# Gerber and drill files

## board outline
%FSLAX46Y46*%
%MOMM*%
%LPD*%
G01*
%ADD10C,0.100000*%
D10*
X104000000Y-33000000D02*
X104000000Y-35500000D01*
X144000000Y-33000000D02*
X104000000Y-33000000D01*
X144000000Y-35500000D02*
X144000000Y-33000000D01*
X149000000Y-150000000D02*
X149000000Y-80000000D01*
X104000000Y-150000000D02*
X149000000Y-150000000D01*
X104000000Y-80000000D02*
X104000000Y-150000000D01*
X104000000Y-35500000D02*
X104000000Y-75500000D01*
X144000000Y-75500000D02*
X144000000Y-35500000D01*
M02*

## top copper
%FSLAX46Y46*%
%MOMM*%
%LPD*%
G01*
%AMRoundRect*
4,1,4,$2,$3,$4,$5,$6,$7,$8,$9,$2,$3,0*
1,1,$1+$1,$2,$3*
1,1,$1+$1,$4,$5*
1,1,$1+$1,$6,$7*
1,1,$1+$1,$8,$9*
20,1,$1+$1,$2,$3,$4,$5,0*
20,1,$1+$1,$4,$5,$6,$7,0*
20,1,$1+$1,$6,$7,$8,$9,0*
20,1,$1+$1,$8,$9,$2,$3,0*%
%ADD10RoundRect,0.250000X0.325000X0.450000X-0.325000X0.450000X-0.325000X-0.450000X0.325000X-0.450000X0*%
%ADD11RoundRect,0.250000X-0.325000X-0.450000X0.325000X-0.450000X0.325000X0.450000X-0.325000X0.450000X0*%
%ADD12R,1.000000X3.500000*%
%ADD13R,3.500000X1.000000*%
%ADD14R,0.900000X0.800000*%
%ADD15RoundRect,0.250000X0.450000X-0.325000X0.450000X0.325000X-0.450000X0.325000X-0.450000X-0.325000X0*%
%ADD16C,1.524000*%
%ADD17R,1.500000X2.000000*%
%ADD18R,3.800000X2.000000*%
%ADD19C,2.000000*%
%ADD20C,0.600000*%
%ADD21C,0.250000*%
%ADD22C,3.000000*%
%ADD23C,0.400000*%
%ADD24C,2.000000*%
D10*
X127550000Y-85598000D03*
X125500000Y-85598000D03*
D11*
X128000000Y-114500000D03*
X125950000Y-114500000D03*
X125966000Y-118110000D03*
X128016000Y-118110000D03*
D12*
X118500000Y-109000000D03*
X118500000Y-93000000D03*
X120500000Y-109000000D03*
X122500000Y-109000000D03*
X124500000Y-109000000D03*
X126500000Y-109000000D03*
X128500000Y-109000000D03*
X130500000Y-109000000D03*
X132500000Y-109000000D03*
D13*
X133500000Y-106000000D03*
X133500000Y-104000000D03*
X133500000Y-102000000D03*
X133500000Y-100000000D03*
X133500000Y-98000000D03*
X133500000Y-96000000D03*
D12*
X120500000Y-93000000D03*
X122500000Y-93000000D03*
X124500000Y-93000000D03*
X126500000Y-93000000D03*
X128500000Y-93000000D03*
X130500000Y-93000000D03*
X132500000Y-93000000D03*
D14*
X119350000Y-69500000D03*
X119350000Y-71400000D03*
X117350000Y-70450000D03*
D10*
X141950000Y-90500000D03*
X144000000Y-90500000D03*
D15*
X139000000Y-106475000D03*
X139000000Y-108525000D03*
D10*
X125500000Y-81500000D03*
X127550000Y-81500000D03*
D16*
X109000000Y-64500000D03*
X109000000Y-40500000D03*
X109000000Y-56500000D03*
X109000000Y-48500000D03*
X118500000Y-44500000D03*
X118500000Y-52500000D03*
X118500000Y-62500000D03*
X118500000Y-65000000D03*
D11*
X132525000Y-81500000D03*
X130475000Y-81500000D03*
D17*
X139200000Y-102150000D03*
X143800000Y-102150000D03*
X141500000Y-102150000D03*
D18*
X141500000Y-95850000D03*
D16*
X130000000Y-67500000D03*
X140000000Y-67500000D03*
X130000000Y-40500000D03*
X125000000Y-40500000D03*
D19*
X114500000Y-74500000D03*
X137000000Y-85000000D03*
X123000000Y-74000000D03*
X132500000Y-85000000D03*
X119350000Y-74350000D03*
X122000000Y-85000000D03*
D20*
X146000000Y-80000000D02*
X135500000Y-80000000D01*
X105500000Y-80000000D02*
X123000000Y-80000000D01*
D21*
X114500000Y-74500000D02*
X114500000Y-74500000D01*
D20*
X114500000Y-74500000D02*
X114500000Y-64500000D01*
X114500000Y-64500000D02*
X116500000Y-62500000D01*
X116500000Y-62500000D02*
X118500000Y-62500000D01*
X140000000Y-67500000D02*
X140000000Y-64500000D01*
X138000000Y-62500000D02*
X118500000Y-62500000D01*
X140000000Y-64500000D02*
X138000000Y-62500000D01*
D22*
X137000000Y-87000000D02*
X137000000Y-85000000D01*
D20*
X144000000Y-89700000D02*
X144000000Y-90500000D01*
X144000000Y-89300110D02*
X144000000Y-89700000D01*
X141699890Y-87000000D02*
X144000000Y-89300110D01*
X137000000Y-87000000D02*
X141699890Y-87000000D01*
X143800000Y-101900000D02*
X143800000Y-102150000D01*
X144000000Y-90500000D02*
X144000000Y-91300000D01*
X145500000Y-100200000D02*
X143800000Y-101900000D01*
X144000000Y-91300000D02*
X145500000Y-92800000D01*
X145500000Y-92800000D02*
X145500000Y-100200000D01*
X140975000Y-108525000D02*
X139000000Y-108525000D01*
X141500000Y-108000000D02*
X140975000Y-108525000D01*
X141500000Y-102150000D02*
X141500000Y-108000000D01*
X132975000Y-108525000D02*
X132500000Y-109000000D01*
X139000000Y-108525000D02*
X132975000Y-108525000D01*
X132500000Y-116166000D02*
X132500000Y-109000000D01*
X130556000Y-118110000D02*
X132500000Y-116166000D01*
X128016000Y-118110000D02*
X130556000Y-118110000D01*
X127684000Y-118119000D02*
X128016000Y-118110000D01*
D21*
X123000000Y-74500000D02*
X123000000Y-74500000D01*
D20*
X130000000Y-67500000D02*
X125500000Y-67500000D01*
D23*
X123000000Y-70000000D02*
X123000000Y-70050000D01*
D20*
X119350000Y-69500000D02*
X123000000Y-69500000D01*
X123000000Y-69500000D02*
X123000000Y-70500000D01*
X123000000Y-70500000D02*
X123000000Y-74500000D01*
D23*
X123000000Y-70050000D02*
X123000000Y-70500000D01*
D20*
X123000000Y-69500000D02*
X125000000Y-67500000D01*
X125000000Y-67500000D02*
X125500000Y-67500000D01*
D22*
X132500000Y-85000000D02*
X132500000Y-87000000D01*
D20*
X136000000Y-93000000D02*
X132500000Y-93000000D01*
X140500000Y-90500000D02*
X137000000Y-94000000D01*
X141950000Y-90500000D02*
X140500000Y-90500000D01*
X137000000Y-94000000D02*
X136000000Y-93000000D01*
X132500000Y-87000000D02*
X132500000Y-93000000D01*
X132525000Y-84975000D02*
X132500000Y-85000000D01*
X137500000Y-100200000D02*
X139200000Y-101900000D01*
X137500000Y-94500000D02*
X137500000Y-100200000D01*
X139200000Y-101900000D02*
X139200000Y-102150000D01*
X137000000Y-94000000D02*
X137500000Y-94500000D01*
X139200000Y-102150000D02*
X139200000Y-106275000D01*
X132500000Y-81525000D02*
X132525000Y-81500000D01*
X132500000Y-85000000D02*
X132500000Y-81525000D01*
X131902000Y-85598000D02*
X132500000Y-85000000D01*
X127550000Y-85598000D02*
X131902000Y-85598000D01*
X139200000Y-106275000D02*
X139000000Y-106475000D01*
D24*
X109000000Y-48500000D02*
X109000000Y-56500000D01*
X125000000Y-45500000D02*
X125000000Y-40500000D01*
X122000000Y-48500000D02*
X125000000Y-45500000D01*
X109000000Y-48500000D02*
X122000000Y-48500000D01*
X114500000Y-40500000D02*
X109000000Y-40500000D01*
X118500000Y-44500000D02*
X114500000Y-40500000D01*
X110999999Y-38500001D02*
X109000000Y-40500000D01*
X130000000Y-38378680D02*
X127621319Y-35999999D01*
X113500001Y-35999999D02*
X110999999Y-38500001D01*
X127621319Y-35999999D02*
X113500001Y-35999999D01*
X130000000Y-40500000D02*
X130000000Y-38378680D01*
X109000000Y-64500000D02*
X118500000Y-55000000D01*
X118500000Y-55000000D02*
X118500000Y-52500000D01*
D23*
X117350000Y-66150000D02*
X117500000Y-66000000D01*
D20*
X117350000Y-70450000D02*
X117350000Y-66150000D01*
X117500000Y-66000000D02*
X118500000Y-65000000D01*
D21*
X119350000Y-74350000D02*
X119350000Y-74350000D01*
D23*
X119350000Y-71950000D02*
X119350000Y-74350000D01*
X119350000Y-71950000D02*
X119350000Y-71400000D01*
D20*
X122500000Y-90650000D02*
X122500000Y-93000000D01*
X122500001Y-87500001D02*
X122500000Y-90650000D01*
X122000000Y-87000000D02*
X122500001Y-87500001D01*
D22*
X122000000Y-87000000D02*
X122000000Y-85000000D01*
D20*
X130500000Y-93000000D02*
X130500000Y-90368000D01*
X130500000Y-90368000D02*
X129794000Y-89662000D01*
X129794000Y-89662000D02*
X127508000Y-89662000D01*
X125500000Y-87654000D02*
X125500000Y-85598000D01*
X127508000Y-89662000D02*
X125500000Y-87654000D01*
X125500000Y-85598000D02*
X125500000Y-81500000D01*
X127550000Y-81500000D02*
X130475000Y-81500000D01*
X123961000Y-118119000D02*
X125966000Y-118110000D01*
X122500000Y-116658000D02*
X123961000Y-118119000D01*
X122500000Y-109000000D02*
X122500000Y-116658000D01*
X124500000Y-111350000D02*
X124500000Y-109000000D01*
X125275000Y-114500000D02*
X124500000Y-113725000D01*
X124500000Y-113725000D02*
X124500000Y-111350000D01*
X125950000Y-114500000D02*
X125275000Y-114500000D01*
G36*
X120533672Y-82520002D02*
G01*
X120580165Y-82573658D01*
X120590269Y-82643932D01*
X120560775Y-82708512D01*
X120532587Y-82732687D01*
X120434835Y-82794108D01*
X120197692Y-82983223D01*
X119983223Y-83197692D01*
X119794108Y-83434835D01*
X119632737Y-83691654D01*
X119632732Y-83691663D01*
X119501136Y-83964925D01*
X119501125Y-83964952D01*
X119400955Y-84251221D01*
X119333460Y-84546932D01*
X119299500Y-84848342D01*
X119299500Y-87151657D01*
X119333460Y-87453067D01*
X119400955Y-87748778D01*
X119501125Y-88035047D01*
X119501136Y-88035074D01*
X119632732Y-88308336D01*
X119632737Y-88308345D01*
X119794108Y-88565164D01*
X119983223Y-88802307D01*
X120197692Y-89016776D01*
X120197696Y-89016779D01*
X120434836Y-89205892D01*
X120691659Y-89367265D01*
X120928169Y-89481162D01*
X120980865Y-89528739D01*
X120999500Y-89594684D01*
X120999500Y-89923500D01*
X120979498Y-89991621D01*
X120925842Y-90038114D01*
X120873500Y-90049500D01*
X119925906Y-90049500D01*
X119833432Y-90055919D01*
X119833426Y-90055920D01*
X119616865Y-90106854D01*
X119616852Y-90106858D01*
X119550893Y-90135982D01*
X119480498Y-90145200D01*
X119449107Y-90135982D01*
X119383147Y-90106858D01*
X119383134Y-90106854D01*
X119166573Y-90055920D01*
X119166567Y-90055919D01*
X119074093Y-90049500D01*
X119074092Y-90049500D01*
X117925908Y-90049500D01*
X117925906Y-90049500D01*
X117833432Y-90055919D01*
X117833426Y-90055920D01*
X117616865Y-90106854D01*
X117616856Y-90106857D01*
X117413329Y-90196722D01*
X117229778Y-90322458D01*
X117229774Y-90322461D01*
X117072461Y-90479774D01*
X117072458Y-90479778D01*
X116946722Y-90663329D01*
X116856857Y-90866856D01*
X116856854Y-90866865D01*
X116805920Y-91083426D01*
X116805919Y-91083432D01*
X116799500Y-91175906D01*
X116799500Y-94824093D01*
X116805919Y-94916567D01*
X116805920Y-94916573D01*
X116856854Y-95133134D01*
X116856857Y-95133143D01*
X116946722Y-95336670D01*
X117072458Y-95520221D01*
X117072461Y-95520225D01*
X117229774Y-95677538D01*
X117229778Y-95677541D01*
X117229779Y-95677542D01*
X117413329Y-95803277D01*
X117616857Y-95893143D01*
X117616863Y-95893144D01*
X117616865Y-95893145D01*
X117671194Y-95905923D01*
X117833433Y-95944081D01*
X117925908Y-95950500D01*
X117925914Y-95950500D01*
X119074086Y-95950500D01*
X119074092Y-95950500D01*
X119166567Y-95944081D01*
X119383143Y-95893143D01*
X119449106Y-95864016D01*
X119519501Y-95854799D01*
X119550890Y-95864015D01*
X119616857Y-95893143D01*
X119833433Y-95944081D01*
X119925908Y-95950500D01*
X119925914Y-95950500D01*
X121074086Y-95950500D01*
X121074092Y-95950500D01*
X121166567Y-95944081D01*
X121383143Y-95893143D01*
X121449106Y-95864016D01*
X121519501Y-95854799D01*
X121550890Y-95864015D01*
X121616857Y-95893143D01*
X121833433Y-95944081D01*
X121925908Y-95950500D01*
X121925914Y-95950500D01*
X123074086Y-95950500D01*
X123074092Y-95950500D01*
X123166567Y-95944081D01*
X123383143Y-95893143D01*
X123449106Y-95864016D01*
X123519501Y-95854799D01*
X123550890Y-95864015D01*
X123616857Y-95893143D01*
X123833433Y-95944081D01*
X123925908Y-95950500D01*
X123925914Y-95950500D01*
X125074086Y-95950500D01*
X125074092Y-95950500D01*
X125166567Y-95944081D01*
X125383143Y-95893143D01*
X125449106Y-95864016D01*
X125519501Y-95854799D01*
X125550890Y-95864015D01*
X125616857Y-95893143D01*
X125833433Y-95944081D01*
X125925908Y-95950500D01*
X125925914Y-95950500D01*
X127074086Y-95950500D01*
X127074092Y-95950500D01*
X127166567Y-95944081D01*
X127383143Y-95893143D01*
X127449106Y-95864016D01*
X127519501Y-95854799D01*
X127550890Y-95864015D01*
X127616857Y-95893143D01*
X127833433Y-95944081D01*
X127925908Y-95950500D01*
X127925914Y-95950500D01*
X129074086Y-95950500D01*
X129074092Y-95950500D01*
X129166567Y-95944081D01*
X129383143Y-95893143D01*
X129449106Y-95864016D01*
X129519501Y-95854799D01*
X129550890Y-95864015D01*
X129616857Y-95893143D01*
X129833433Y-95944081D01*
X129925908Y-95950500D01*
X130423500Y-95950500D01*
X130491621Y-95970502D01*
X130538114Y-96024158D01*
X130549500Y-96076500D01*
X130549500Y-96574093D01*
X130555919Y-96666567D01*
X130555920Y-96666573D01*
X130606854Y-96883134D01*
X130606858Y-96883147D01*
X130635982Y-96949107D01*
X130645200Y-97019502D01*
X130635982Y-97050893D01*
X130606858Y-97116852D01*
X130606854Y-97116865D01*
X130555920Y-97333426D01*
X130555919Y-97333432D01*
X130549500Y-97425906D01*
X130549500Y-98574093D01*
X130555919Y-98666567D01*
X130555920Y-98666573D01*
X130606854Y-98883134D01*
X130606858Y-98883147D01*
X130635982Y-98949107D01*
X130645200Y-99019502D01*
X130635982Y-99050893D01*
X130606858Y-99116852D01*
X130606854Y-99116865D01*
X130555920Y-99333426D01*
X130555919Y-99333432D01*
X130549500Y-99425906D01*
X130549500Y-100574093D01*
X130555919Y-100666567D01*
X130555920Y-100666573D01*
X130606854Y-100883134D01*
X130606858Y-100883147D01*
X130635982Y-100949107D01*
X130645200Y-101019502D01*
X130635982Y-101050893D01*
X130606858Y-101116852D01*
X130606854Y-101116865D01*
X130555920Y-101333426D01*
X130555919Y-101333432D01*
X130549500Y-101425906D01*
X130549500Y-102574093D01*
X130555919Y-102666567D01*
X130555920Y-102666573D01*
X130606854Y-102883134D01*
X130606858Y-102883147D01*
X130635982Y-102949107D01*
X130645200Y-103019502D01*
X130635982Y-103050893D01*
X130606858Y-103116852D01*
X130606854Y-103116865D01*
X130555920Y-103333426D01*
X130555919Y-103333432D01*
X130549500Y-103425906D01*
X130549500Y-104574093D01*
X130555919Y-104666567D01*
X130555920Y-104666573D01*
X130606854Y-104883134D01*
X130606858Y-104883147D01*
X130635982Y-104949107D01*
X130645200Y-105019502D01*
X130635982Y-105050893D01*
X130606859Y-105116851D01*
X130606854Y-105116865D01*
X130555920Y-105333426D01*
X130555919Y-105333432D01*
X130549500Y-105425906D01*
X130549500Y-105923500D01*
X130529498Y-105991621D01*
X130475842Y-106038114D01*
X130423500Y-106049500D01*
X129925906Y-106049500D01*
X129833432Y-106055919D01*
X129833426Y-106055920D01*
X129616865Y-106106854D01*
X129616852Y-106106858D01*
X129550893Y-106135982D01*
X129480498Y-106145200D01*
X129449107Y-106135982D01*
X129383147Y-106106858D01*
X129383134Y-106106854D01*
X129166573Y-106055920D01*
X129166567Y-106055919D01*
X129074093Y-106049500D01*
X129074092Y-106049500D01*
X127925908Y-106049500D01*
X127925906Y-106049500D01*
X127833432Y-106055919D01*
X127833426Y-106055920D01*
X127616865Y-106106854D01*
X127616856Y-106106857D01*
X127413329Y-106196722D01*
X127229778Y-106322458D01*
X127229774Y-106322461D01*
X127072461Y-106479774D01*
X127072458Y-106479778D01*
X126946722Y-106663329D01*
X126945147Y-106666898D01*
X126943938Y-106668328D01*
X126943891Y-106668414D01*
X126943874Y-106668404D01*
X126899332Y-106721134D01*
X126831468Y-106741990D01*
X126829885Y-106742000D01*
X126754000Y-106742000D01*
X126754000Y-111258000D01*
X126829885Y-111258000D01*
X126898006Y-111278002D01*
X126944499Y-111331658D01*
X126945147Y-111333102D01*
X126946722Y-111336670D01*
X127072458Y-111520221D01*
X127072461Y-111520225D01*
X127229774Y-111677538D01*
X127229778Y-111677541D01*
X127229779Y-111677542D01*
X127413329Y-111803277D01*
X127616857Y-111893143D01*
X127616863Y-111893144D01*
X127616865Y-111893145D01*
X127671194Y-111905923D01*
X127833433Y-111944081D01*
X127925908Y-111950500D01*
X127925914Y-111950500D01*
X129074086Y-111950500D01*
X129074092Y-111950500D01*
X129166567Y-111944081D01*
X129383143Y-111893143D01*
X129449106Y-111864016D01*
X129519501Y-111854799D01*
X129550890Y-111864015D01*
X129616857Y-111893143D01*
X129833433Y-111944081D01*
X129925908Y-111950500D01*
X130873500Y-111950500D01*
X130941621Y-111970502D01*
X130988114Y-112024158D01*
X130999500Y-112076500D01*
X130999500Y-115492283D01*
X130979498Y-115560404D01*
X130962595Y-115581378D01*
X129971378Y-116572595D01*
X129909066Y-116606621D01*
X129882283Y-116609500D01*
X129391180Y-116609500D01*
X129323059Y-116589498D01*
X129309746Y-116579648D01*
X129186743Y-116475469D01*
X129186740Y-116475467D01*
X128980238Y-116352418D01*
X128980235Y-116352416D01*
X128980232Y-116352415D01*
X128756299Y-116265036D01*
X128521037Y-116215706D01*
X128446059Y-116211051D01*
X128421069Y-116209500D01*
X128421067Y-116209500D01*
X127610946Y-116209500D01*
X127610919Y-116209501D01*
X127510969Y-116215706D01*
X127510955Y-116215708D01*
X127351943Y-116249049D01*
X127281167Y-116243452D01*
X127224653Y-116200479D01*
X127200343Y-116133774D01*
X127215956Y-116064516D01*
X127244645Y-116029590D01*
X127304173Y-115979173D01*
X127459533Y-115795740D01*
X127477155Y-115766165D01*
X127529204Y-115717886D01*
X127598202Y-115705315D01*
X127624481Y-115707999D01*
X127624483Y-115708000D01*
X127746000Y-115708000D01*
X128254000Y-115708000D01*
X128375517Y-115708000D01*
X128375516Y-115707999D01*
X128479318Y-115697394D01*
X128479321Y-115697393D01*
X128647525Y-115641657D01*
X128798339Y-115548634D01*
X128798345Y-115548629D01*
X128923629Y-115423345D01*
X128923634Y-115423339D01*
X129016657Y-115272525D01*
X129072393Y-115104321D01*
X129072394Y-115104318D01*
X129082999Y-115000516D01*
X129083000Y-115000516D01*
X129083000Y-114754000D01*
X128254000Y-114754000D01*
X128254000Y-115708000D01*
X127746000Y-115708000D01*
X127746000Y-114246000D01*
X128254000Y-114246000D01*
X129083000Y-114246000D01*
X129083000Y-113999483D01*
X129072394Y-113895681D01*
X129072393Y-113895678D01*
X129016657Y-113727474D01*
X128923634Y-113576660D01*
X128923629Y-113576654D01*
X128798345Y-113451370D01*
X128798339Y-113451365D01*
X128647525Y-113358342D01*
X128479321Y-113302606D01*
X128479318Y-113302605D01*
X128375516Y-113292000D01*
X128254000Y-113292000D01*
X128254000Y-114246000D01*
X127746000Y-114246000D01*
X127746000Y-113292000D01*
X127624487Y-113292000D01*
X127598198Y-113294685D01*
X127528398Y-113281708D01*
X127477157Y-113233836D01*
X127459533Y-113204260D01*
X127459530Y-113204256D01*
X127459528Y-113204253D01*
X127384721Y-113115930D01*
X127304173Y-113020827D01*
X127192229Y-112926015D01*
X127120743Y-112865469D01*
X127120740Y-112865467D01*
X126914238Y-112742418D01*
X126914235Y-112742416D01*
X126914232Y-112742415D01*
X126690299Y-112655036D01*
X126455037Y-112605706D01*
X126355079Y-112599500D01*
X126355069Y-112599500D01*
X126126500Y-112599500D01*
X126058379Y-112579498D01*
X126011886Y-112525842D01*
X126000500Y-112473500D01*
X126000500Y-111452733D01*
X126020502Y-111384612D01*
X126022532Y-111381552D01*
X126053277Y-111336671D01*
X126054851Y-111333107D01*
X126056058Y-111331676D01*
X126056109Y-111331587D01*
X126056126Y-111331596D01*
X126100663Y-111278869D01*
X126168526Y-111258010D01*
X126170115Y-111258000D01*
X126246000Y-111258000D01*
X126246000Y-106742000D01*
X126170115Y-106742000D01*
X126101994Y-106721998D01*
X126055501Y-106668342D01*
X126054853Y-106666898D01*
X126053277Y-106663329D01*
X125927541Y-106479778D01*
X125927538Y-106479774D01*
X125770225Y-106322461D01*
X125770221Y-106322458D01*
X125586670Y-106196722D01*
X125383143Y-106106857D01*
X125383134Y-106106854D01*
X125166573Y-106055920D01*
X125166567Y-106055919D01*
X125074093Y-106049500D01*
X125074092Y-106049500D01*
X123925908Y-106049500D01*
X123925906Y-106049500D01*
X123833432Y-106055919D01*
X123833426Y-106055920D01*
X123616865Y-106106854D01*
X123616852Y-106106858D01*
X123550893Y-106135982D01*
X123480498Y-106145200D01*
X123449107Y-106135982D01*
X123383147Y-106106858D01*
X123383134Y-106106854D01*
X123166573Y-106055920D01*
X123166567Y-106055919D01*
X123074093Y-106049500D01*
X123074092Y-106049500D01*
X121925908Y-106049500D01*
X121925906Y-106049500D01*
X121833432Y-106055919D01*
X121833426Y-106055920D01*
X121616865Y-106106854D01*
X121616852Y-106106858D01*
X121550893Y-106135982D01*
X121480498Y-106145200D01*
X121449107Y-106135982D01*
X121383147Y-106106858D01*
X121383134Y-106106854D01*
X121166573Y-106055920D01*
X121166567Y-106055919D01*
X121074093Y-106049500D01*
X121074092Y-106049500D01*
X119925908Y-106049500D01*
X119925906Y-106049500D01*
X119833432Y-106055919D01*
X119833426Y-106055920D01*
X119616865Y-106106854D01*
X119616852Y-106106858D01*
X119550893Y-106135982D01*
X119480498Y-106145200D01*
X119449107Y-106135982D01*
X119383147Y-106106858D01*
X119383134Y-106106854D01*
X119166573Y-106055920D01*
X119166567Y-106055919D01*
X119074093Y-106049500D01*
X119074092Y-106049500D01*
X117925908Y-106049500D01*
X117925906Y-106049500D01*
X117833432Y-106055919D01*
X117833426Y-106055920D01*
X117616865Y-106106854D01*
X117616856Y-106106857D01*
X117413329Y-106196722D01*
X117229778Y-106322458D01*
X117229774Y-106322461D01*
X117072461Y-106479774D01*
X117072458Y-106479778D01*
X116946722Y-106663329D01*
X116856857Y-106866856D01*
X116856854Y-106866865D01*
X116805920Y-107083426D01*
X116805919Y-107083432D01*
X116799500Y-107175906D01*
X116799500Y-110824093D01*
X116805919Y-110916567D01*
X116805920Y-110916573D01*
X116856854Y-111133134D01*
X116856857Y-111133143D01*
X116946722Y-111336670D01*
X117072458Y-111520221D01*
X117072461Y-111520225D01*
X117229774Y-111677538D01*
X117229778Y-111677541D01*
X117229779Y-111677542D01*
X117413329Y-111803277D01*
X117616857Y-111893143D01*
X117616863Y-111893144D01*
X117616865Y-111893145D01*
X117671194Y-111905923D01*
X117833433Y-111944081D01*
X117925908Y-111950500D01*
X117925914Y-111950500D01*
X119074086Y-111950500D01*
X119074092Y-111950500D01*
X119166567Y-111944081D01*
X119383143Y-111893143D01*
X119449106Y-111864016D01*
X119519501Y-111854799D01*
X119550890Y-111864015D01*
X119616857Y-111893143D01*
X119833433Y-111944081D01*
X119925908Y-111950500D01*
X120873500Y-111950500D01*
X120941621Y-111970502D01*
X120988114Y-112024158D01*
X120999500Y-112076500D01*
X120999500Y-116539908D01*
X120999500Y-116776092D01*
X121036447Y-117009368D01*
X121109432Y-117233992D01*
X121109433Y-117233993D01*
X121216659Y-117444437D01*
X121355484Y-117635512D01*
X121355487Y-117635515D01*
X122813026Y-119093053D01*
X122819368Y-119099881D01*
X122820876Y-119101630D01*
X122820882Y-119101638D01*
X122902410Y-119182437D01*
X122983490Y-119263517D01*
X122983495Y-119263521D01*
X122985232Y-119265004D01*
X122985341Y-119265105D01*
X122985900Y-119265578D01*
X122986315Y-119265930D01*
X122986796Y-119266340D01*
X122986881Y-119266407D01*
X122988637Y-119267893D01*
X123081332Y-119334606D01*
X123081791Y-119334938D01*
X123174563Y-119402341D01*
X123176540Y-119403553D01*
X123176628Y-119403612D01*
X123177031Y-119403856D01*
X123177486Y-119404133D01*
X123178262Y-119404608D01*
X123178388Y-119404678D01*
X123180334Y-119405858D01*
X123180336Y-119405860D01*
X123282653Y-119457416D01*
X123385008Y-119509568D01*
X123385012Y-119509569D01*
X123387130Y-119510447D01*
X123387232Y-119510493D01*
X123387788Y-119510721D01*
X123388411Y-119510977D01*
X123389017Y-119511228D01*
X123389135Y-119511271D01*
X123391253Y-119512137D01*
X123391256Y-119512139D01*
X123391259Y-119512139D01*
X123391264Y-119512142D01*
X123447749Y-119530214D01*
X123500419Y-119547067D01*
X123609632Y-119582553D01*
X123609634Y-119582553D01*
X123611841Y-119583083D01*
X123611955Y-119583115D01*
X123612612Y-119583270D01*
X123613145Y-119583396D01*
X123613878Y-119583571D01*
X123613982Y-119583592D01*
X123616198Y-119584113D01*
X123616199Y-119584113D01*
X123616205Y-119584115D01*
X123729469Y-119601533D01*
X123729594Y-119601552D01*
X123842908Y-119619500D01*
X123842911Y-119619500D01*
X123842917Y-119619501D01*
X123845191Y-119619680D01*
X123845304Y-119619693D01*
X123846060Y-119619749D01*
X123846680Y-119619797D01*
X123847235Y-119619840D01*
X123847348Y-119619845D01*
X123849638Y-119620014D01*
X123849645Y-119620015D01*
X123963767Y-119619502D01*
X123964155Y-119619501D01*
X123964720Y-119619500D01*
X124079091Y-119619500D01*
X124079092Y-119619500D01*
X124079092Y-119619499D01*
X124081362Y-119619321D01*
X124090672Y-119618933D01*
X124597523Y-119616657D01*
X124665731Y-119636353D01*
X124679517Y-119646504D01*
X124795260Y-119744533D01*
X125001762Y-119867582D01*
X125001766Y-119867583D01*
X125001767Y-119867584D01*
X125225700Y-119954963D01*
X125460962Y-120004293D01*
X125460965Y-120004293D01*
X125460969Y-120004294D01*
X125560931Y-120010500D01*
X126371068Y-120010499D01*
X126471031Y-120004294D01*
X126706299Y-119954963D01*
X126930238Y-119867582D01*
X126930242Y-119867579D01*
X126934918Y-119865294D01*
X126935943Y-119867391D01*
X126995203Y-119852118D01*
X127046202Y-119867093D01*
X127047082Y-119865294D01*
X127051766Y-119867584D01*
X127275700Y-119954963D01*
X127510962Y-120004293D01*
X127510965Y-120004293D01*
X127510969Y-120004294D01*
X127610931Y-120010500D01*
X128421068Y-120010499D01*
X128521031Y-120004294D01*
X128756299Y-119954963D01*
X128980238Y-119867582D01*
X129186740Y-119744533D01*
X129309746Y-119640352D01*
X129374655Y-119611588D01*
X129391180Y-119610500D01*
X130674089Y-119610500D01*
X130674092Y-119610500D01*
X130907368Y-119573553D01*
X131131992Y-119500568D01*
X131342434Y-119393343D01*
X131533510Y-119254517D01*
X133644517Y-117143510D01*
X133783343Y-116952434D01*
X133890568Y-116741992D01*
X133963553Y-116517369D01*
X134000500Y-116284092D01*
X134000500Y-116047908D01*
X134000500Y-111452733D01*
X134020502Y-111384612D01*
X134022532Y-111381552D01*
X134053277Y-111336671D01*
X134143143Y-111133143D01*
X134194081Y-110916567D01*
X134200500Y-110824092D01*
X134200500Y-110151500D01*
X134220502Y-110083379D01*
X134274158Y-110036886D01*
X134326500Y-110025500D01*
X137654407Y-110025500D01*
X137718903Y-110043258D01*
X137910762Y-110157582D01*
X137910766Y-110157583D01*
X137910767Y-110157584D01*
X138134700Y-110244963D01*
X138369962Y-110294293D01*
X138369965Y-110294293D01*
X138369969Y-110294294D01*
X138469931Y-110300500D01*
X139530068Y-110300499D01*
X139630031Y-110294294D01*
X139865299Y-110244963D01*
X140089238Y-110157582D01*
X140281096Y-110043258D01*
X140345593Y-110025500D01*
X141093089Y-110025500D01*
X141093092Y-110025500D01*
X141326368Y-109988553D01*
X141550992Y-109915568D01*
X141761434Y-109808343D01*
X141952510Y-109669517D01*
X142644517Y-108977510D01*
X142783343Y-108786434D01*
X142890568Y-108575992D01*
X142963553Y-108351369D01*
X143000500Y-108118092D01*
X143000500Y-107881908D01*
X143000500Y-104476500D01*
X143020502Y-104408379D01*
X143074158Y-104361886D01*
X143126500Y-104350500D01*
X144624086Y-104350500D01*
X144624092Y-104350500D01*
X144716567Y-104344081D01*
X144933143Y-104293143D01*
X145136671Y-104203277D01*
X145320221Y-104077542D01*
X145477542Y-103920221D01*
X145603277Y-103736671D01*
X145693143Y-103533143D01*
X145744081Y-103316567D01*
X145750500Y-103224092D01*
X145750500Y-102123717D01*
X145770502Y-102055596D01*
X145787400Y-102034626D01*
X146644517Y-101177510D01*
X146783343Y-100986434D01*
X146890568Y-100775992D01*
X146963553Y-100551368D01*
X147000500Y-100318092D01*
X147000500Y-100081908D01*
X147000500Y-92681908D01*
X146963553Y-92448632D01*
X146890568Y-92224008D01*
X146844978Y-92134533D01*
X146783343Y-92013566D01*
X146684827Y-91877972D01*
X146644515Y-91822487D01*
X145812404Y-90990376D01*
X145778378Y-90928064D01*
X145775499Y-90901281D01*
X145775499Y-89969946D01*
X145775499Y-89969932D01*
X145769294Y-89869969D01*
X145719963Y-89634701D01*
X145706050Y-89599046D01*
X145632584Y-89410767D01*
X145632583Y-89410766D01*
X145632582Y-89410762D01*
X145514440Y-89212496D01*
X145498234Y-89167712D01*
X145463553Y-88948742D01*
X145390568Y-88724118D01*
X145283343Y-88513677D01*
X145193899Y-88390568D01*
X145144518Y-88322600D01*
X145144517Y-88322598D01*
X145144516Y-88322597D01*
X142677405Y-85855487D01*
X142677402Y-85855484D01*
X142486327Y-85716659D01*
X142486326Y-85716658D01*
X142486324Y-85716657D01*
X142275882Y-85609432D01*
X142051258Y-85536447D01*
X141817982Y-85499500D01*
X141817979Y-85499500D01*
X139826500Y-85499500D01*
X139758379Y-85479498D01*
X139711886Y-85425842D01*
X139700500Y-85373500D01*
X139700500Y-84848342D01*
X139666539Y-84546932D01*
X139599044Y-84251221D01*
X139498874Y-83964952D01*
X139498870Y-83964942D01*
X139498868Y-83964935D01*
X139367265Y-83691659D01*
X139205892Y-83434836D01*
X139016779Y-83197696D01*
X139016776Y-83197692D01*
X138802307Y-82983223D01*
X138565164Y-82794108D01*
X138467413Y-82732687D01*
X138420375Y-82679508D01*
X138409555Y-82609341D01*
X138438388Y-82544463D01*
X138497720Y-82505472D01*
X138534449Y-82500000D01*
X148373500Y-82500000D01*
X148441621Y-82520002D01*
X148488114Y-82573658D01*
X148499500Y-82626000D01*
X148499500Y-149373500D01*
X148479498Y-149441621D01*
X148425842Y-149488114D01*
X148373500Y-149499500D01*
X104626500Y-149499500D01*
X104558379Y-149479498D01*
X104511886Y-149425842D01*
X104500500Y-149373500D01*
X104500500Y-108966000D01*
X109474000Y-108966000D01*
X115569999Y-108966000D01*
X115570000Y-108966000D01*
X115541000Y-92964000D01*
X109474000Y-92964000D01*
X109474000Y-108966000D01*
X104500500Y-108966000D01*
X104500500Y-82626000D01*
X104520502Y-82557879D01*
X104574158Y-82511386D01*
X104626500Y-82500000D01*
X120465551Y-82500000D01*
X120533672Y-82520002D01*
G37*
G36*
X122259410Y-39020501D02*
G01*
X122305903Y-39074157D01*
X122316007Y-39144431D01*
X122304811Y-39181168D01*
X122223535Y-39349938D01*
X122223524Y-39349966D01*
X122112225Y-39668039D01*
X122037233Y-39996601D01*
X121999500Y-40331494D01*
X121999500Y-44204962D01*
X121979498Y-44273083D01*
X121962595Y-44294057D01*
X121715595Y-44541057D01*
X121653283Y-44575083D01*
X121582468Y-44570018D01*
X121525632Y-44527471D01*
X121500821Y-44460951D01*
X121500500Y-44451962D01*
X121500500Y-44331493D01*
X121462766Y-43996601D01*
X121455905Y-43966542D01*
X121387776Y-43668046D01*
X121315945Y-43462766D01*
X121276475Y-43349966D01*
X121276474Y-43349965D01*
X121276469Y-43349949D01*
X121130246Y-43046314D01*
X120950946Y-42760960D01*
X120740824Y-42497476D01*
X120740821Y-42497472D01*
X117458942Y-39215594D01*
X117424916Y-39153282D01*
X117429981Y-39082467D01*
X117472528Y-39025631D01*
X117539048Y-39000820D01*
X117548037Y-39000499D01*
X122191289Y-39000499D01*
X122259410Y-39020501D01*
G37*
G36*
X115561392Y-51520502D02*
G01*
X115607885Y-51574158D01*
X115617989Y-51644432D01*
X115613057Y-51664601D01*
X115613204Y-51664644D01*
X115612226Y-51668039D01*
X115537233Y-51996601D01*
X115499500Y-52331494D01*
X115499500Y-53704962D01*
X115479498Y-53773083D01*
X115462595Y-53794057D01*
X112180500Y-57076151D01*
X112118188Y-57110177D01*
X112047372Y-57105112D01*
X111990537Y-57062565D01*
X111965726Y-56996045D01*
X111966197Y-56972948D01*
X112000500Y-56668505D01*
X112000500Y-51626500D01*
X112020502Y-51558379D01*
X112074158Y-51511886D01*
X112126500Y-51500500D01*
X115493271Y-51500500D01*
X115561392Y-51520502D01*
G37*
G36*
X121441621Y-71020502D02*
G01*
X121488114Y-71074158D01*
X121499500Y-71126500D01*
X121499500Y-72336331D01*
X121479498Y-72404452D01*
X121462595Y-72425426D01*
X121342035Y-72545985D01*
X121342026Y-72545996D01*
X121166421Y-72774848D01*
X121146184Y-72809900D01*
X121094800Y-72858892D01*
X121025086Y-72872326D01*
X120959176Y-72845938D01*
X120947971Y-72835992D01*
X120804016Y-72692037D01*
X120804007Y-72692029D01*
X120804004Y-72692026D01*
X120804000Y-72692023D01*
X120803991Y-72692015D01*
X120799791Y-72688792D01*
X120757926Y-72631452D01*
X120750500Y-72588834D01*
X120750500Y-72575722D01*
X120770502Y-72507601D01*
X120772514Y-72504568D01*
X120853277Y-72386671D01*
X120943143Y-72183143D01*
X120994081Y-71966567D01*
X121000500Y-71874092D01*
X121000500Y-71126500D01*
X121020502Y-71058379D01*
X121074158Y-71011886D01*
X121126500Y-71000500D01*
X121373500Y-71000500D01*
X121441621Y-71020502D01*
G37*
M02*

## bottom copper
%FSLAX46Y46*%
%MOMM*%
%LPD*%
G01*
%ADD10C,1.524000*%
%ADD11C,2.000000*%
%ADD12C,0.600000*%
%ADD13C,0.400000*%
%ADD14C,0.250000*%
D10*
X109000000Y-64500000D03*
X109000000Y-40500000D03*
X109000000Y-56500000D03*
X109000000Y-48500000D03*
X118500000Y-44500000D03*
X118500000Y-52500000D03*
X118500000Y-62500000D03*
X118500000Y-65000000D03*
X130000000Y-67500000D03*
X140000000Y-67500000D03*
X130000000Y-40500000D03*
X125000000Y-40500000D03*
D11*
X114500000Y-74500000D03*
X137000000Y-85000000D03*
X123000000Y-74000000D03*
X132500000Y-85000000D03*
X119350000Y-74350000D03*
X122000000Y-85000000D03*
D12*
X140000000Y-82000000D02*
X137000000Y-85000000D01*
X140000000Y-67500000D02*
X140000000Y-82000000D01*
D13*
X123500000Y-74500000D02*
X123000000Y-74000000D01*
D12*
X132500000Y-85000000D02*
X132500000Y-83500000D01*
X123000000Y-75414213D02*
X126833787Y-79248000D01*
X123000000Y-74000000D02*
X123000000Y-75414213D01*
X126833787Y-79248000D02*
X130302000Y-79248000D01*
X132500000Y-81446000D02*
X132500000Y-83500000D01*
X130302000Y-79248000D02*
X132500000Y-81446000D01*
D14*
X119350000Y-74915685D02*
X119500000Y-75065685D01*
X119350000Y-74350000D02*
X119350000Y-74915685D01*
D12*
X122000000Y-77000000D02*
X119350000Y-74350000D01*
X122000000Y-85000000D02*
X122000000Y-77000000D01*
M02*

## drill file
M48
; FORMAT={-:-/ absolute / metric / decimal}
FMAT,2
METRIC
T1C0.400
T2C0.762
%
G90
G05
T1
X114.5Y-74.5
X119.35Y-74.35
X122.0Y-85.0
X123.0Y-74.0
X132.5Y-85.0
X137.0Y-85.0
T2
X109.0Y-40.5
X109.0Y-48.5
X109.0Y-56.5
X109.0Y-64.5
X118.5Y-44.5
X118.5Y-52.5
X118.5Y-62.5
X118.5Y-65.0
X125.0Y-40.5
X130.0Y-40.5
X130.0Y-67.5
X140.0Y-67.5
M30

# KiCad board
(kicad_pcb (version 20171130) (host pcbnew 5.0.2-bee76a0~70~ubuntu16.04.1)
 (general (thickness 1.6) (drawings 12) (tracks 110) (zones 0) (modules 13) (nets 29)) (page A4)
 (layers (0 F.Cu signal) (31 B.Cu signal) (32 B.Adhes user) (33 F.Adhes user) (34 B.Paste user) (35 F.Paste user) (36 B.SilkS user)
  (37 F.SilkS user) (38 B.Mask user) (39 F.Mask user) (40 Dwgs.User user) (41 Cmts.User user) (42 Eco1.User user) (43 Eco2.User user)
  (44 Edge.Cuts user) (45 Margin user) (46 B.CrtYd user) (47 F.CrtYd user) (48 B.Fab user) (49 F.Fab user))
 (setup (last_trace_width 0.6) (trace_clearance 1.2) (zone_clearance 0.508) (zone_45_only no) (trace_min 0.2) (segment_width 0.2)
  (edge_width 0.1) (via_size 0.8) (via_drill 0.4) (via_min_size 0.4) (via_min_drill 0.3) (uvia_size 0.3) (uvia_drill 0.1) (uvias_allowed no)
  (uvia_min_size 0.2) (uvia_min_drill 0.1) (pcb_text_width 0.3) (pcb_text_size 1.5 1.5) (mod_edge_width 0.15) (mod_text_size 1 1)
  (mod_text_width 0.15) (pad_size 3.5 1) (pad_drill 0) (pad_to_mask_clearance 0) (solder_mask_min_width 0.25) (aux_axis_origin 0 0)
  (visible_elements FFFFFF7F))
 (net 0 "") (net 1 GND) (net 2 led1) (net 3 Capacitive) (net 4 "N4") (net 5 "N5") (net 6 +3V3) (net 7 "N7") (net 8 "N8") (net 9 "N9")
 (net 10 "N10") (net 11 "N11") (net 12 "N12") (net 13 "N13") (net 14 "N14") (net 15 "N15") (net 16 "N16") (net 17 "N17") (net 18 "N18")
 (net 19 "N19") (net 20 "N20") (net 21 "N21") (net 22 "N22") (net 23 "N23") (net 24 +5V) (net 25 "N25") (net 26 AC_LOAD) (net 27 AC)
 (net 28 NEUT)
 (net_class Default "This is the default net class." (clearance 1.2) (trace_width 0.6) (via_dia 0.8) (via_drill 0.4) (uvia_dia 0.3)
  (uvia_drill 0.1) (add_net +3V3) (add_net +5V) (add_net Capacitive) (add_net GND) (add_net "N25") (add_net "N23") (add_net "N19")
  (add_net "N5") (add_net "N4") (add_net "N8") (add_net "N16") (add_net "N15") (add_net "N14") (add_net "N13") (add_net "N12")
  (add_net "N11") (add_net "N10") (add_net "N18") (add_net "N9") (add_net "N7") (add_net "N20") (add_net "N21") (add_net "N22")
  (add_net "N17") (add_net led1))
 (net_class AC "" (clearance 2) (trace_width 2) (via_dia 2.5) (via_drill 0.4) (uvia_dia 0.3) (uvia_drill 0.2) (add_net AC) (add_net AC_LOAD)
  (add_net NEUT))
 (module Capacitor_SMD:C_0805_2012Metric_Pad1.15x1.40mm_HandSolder (layer F.Cu) (at 126.525 85.598 180)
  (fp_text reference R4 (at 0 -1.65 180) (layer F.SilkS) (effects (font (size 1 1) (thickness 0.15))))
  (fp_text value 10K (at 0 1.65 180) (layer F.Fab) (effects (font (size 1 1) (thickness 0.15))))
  (pad 1 smd roundrect (at -1.025 0 180) (size 1.15 1.4) (layers F.Cu F.Paste F.Mask) (roundrect_rratio 0.217391) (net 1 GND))
  (pad 2 smd roundrect (at 1.025 0 180) (size 1.15 1.4) (layers F.Cu F.Paste F.Mask) (roundrect_rratio 0.217391) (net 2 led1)))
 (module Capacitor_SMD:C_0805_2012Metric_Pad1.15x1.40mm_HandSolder (layer F.Cu) (at 126.975 114.5)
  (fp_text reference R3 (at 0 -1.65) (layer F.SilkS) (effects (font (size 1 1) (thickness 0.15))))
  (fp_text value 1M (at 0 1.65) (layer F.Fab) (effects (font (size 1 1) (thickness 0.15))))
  (pad 2 smd roundrect (at 1.025 0) (size 1.15 1.4) (layers F.Cu F.Paste F.Mask) (roundrect_rratio 0.217391) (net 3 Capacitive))
  (pad 1 smd roundrect (at -1.025 0) (size 1.15 1.4) (layers F.Cu F.Paste F.Mask) (roundrect_rratio 0.217391) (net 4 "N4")))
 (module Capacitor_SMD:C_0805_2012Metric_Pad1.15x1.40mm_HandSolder (layer F.Cu) (at 126.991 118.11)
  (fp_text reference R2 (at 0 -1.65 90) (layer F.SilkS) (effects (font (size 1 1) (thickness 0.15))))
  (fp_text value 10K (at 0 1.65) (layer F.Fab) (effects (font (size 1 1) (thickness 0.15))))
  (pad 1 smd roundrect (at -1.025 0) (size 1.15 1.4) (layers F.Cu F.Paste F.Mask) (roundrect_rratio 0.217391) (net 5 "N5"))
  (pad 2 smd roundrect (at 1.025 0) (size 1.15 1.4) (layers F.Cu F.Paste F.Mask) (roundrect_rratio 0.217391) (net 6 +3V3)))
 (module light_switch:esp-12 (layer F.Cu) (at 125.5 101 90)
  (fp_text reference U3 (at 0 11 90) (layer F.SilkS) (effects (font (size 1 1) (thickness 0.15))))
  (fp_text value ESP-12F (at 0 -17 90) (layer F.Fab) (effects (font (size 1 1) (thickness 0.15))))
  (pad 22 smd rect (at -8 -7 90) (size 3.5 1) (layers F.Cu F.Paste F.Mask) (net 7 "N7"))
  (pad 1 smd rect (at 8 -7 90) (size 3.5 1) (layers F.Cu F.Paste F.Mask) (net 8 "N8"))
  (pad 21 smd rect (at -8 -5 90) (size 3.5 1) (layers F.Cu F.Paste F.Mask) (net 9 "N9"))
  (pad 20 smd rect (at -8 -3 90) (size 3.5 1) (layers F.Cu F.Paste F.Mask) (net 5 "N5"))
  (pad 19 smd rect (at -8 -1 90) (size 3.5 1) (layers F.Cu F.Paste F.Mask) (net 4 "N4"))
  (pad 18 smd rect (at -8 1 90) (size 3.5 1) (layers F.Cu F.Paste F.Mask) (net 3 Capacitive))
  (pad 17 smd rect (at -8 3 90) (size 3.5 1) (layers F.Cu F.Paste F.Mask) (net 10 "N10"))
  (pad 16 smd rect (at -8 5 90) (size 3.5 1) (layers F.Cu F.Paste F.Mask) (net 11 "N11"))
  (pad 15 smd rect (at -8 7 90) (size 3.5 1) (layers F.Cu F.Paste F.Mask) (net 6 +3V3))
  (pad 14 smd rect (at -5 8) (size 3.5 1) (layers F.Cu F.Paste F.Mask) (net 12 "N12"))
  (pad 13 smd rect (at -3 8) (size 3.5 1) (layers F.Cu F.Paste F.Mask) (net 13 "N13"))
  (pad 12 smd rect (at -1 8) (size 3.5 1) (layers F.Cu F.Paste F.Mask) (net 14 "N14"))
  (pad 11 smd rect (at 1 8) (size 3.5 1) (layers F.Cu F.Paste F.Mask) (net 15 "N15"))
  (pad 10 smd rect (at 3 8) (size 3.5 1) (layers F.Cu F.Paste F.Mask) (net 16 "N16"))
  (pad 9 smd rect (at 5 8 180) (size 3.5 1) (layers F.Cu F.Paste F.Mask) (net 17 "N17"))
  (pad 2 smd rect (at 8 -5 90) (size 3.5 1) (layers F.Cu F.Paste F.Mask) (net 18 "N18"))
  (pad 3 smd rect (at 8 -3 90) (size 3.5 1) (layers F.Cu F.Paste F.Mask) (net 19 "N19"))
  (pad 4 smd rect (at 8 -1 90) (size 3.5 1) (layers F.Cu F.Paste F.Mask) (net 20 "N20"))
  (pad 5 smd rect (at 8 1 90) (size 3.5 1) (layers F.Cu F.Paste F.Mask) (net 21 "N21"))
  (pad 6 smd rect (at 8 3 90) (size 3.5 1) (layers F.Cu F.Paste F.Mask) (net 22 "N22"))
  (pad 7 smd rect (at 8 5 90) (size 3.5 1) (layers F.Cu F.Paste F.Mask) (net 2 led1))
  (pad 8 smd rect (at 8 7 90) (size 3.5 1) (layers F.Cu F.Paste F.Mask) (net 1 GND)))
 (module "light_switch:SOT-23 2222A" (layer F.Cu) (at 119 70.45 90)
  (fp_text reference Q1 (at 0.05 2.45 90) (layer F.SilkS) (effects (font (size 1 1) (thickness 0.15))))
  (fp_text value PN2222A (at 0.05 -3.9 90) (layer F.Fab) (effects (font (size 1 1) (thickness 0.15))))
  (pad 1 smd rect (at 0.95 0.35 90) (size 0.8 0.9) (layers F.Cu F.Paste F.Mask) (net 1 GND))
  (pad 2 smd rect (at -0.95 0.35 90) (size 0.8 0.9) (layers F.Cu F.Paste F.Mask) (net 19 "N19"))
  (pad 3 smd rect (at 0 -1.65 90) (size 0.8 0.9) (layers F.Cu F.Paste F.Mask) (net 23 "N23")))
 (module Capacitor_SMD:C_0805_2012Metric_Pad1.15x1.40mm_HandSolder (layer F.Cu) (at 142.975 90.5 180)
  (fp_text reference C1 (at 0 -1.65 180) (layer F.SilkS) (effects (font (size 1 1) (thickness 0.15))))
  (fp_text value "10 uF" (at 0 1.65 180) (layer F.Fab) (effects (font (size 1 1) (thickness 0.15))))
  (pad 2 smd roundrect (at 1.025 0 180) (size 1.15 1.4) (layers F.Cu F.Paste F.Mask) (roundrect_rratio 0.217391) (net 1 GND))
  (pad 1 smd roundrect (at -1.025 0 180) (size 1.15 1.4) (layers F.Cu F.Paste F.Mask) (roundrect_rratio 0.217391) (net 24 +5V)))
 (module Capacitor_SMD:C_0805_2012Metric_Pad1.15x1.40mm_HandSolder (layer F.Cu) (at 139 107.5 90)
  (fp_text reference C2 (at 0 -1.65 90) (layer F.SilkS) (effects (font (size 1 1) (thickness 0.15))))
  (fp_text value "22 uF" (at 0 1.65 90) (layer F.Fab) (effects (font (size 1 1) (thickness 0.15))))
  (pad 2 smd roundrect (at 1.025 0 90) (size 1.15 1.4) (layers F.Cu F.Paste F.Mask) (roundrect_rratio 0.217391) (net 1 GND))
  (pad 1 smd roundrect (at -1.025 0 90) (size 1.15 1.4) (layers F.Cu F.Paste F.Mask) (roundrect_rratio 0.217391) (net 6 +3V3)))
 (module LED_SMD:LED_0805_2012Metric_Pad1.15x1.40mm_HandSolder (layer F.Cu) (at 126.525 81.5 180)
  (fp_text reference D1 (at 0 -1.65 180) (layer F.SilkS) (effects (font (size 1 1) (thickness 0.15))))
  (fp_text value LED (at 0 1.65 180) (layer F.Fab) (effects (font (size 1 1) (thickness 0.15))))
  (pad 2 smd roundrect (at 1.025 0 180) (size 1.15 1.4) (layers F.Cu F.Paste F.Mask) (roundrect_rratio 0.217391) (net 2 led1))
  (pad 1 smd roundrect (at -1.025 0 180) (size 1.15 1.4) (layers F.Cu F.Paste F.Mask) (roundrect_rratio 0.217391) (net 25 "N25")))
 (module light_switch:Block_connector (layer F.Cu) (at 109 52.5 270)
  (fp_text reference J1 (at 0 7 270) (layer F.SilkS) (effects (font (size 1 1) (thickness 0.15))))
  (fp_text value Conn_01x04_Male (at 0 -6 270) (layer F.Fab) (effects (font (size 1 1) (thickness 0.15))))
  (pad 4 thru_hole circle (at 12 0 270) (size 1.524 1.524) (drill 0.762) (layers *.Cu *.Mask) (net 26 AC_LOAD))
  (pad 1 thru_hole circle (at -12 0 270) (size 1.524 1.524) (drill 0.762) (layers *.Cu *.Mask) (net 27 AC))
  (pad 3 thru_hole circle (at 4 0 270) (size 1.524 1.524) (drill 0.762) (layers *.Cu *.Mask) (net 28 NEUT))
  (pad 2 thru_hole circle (at -4 0 270) (size 1.524 1.524) (drill 0.762) (layers *.Cu *.Mask) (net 28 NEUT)))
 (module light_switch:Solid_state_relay (layer F.Cu) (at 117.5 55 90)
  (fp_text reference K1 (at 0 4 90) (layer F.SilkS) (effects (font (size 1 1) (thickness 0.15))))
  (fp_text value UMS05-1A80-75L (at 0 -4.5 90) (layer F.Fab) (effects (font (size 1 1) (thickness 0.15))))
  (pad 4 thru_hole circle (at 10.5 1 90) (size 1.524 1.524) (drill 0.762) (layers *.Cu *.Mask) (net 27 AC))
  (pad 3 thru_hole circle (at 2.5 1 90) (size 1.524 1.524) (drill 0.762) (layers *.Cu *.Mask) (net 26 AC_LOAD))
  (pad 2 thru_hole circle (at -7.5 1 90) (size 1.524 1.524) (drill 0.762) (layers *.Cu *.Mask) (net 24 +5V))
  (pad 1 thru_hole circle (at -10 1 90) (size 1.524 1.524) (drill 0.762) (layers *.Cu *.Mask) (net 23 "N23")))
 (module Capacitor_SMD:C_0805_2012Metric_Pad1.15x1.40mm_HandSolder (layer F.Cu) (at 131.5 81.5)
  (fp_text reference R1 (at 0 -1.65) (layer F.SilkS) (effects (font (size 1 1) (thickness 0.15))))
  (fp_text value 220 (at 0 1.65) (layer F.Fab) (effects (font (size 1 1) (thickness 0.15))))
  (pad 2 smd roundrect (at 1.025 0) (size 1.15 1.4) (layers F.Cu F.Paste F.Mask) (roundrect_rratio 0.217391) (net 1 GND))
  (pad 1 smd roundrect (at -1.025 0) (size 1.15 1.4) (layers F.Cu F.Paste F.Mask) (roundrect_rratio 0.217391) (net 25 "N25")))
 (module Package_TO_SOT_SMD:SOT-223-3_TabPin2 (layer F.Cu) (at 141.5 99 90)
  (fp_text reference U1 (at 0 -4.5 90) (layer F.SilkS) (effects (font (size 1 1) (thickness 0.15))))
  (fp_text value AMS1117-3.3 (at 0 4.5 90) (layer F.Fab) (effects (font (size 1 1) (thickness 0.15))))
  (pad 1 smd rect (at -3.15 -2.3 90) (size 2 1.5) (layers F.Cu F.Paste F.Mask) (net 1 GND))
  (pad 3 smd rect (at -3.15 2.3 90) (size 2 1.5) (layers F.Cu F.Paste F.Mask) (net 24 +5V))
  (pad 2 smd rect (at -3.15 0 90) (size 2 1.5) (layers F.Cu F.Paste F.Mask) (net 6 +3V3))
  (pad 2 smd rect (at 3.15 0 90) (size 2 3.8) (layers F.Cu F.Paste F.Mask) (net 6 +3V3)))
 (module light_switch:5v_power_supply (layer B.Cu) (at 132.5 54 270)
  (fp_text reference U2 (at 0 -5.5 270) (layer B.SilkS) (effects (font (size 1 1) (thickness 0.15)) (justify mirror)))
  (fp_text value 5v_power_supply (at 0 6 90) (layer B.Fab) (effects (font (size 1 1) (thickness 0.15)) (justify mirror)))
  (pad 4 thru_hole circle (at 13.5 2.5 270) (size 1.524 1.524) (drill 0.762) (layers *.Cu *.Mask) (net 1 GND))
  (pad 3 thru_hole circle (at 13.5 -7.5 270) (size 1.524 1.524) (drill 0.762) (layers *.Cu *.Mask) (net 24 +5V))
  (pad 1 thru_hole circle (at -13.5 2.5 270) (size 1.524 1.524) (drill 0.762) (layers *.Cu *.Mask) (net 27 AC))
  (pad 2 thru_hole circle (at -13.5 7.5 270) (size 1.524 1.524) (drill 0.762) (layers *.Cu *.Mask) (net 28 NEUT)))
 (gr_line (start 104 33) (end 104 35.5) (layer Edge.Cuts) (width 0.1))
 (gr_line (start 144 33) (end 104 33) (layer Edge.Cuts) (width 0.1))
 (gr_line (start 144 35.5) (end 144 33) (layer Edge.Cuts) (width 0.1))
 (gr_line (start 149 150) (end 149 80) (layer Edge.Cuts) (width 0.1))
 (gr_line (start 104 150) (end 149 150) (layer Edge.Cuts) (width 0.1))
 (gr_line (start 104 80) (end 104 150) (layer Edge.Cuts) (width 0.1))
 (gr_line (start 104 35.5) (end 104 75.5) (layer Edge.Cuts) (width 0.1))
 (gr_line (start 144 75.5) (end 144 35.5) (layer Edge.Cuts) (width 0.1))
 (segment (start 146 80) (end 135.5 80) (width 0.6) (layer F.Cu) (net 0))
 (segment (start 105.5 80) (end 123 80) (width 0.6) (layer F.Cu) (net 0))
 (segment (start 114.5 74.5) (end 114.5 74.5) (width 0.25) (layer F.Cu) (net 24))
 (via (at 114.5 74.5) (size 2) (drill 0.4) (layers F.Cu B.Cu) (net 24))
 (via (at 137 85) (size 2) (drill 0.4) (layers F.Cu B.Cu) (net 24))
 (segment (start 114.5 74.5) (end 114.5 64.5) (width 0.6) (layer F.Cu) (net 24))
 (segment (start 114.5 64.5) (end 116.5 62.5) (width 0.6) (layer F.Cu) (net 24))
 (segment (start 116.5 62.5) (end 118.5 62.5) (width 0.6) (layer F.Cu) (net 24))
 (segment (start 140 67.5) (end 140 64.5) (width 0.6) (layer F.Cu) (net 24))
 (segment (start 138 62.5) (end 118.5 62.5) (width 0.6) (layer F.Cu) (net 24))
 (segment (start 140 64.5) (end 138 62.5) (width 0.6) (layer F.Cu) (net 24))
 (segment (start 137 87) (end 137 85) (width 3) (layer F.Cu) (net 24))
 (segment (start 144 89.7) (end 144 90.5) (width 0.6) (layer F.Cu) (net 24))
 (segment (start 144 89.30011) (end 144 89.7) (width 0.6) (layer F.Cu) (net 24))
 (segment (start 141.69989 87) (end 144 89.30011) (width 0.6) (layer F.Cu) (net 24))
 (segment (start 137 87) (end 141.69989 87) (width 0.6) (layer F.Cu) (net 24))
 (segment (start 140 82) (end 137 85) (width 0.6) (layer B.Cu) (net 24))
 (segment (start 140 67.5) (end 140 82) (width 0.6) (layer B.Cu) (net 24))
 (segment (start 143.8 101.9) (end 143.8 102.15) (width 0.6) (layer F.Cu) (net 24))
 (segment (start 144 90.5) (end 144 91.3) (width 0.6) (layer F.Cu) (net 24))
 (segment (start 145.5 100.2) (end 143.8 101.9) (width 0.6) (layer F.Cu) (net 24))
 (segment (start 144 91.3) (end 145.5 92.8) (width 0.6) (layer F.Cu) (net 24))
 (segment (start 145.5 92.8) (end 145.5 100.2) (width 0.6) (layer F.Cu) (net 24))
 (segment (start 140.975 108.525) (end 139 108.525) (width 0.6) (layer F.Cu) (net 6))
 (segment (start 141.5 108) (end 140.975 108.525) (width 0.6) (layer F.Cu) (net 6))
 (segment (start 141.5 102.15) (end 141.5 108) (width 0.6) (layer F.Cu) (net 6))
 (segment (start 132.975 108.525) (end 132.5 109) (width 0.6) (layer F.Cu) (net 6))
 (segment (start 139 108.525) (end 132.975 108.525) (width 0.6) (layer F.Cu) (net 6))
 (segment (start 132.5 116.166) (end 132.5 109) (width 0.6) (layer F.Cu) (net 6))
 (segment (start 130.556 118.11) (end 132.5 116.166) (width 0.6) (layer F.Cu) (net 6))
 (segment (start 128.016 118.11) (end 130.556 118.11) (width 0.6) (layer F.Cu) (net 6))
 (segment (start 127.684 118.119) (end 128.016 118.11) (width 0.6) (layer F.Cu) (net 6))
 (segment (start 123 74.5) (end 123 74.5) (width 0.25) (layer F.Cu) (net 1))
 (via (at 123 74) (size 2) (drill 0.4) (layers F.Cu B.Cu) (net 1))
 (via (at 132.5 85) (size 2) (drill 0.4) (layers F.Cu B.Cu) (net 1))
 (segment (start 123.5 74.5) (end 123 74) (width 0.4) (layer B.Cu) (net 1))
 (segment (start 130 67.5) (end 125.5 67.5) (width 0.6) (layer F.Cu) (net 1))
 (segment (start 123 70) (end 123 70.05) (width 0.4) (layer F.Cu) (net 1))
 (segment (start 119.35 69.5) (end 123 69.5) (width 0.6) (layer F.Cu) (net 1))
 (segment (start 123 69.5) (end 123 70.5) (width 0.6) (layer F.Cu) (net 1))
 (segment (start 123 70.5) (end 123 74.5) (width 0.6) (layer F.Cu) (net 1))
 (segment (start 123 70.05) (end 123 70.5) (width 0.4) (layer F.Cu) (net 1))
 (segment (start 123 69.5) (end 125 67.5) (width 0.6) (layer F.Cu) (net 1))
 (segment (start 125 67.5) (end 125.5 67.5) (width 0.6) (layer F.Cu) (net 1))
 (segment (start 132.5 85) (end 132.5 87) (width 3) (layer F.Cu) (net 1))
 (segment (start 136 93) (end 132.5 93) (width 0.6) (layer F.Cu) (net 1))
 (segment (start 140.5 90.5) (end 137 94) (width 0.6) (layer F.Cu) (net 1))
 (segment (start 141.95 90.5) (end 140.5 90.5) (width 0.6) (layer F.Cu) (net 1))
 (segment (start 137 94) (end 136 93) (width 0.6) (layer F.Cu) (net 1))
 (segment (start 132.5 87) (end 132.5 93) (width 0.6) (layer F.Cu) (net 1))
 (segment (start 132.525 84.975) (end 132.5 85) (width 0.6) (layer F.Cu) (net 1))
 (segment (start 132.5 85) (end 132.5 83.5) (width 0.6) (layer B.Cu) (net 1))
 (segment (start 137.5 100.2) (end 139.2 101.9) (width 0.6) (layer F.Cu) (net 1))
 (segment (start 137.5 94.5) (end 137.5 100.2) (width 0.6) (layer F.Cu) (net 1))
 (segment (start 139.2 101.9) (end 139.2 102.15) (width 0.6) (layer F.Cu) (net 1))
 (segment (start 137 94) (end 137.5 94.5) (width 0.6) (layer F.Cu) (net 1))
 (segment (start 139.2 102.15) (end 139.2 106.275) (width 0.6) (layer F.Cu) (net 1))
 (segment (start 132.5 81.525) (end 132.525 81.5) (width 0.6) (layer F.Cu) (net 1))
 (segment (start 132.5 85) (end 132.5 81.525) (width 0.6) (layer F.Cu) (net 1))
 (segment (start 123 75.414213) (end 126.833787 79.248) (width 0.6) (layer B.Cu) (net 1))
 (segment (start 123 74) (end 123 75.414213) (width 0.6) (layer B.Cu) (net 1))
 (segment (start 126.833787 79.248) (end 130.302 79.248) (width 0.6) (layer B.Cu) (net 1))
 (segment (start 132.5 81.446) (end 132.5 83.5) (width 0.6) (layer B.Cu) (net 1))
 (segment (start 130.302 79.248) (end 132.5 81.446) (width 0.6) (layer B.Cu) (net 1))
 (segment (start 131.902 85.598) (end 132.5 85) (width 0.6) (layer F.Cu) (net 1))
 (segment (start 127.55 85.598) (end 131.902 85.598) (width 0.6) (layer F.Cu) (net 1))
 (segment (start 139.2 106.275) (end 139 106.475) (width 0.6) (layer F.Cu) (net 1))
 (segment (start 109 48.5) (end 109 56.5) (width 2) (layer F.Cu) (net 28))
 (segment (start 125 45.5) (end 125 40.5) (width 2) (layer F.Cu) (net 28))
 (segment (start 122 48.5) (end 125 45.5) (width 2) (layer F.Cu) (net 28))
 (segment (start 109 48.5) (end 122 48.5) (width 2) (layer F.Cu) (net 28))
 (segment (start 114.5 40.5) (end 109 40.5) (width 2) (layer F.Cu) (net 27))
 (segment (start 118.5 44.5) (end 114.5 40.5) (width 2) (layer F.Cu) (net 27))
 (segment (start 110.999999 38.500001) (end 109 40.5) (width 2) (layer F.Cu) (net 27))
 (segment (start 130 38.37868) (end 127.621319 35.999999) (width 2) (layer F.Cu) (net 27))
 (segment (start 113.500001 35.999999) (end 110.999999 38.500001) (width 2) (layer F.Cu) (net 27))
 (segment (start 127.621319 35.999999) (end 113.500001 35.999999) (width 2) (layer F.Cu) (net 27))
 (segment (start 130 40.5) (end 130 38.37868) (width 2) (layer F.Cu) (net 27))
 (segment (start 109 64.5) (end 118.5 55) (width 2) (layer F.Cu) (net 26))
 (segment (start 118.5 55) (end 118.5 52.5) (width 2) (layer F.Cu) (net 26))
 (segment (start 117.35 66.15) (end 117.5 66) (width 0.4) (layer F.Cu) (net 23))
 (segment (start 117.35 70.45) (end 117.35 66.15) (width 0.6) (layer F.Cu) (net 23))
 (segment (start 117.5 66) (end 118.5 65) (width 0.6) (layer F.Cu) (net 23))
 (segment (start 119.35 74.35) (end 119.35 74.35) (width 0.25) (layer F.Cu) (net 19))
 (via (at 119.35 74.35) (size 2) (drill 0.4) (layers F.Cu B.Cu) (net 19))
 (segment (start 119.35 74.915685) (end 119.5 75.065685) (width 0.25) (layer B.Cu) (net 19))
 (segment (start 119.35 74.35) (end 119.35 74.915685) (width 0.25) (layer B.Cu) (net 19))
 (via (at 122 85) (size 2) (drill 0.4) (layers F.Cu B.Cu) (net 19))
 (segment (start 119.35 71.95) (end 119.35 74.35) (width 0.4) (layer F.Cu) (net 19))
 (segment (start 119.35 71.95) (end 119.35 71.4) (width 0.4) (layer F.Cu) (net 19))
 (segment (start 122 77) (end 119.35 74.35) (width 0.6) (layer B.Cu) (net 19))
 (segment (start 122 85) (end 122 77) (width 0.6) (layer B.Cu) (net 19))
 (segment (start 122.5 90.65) (end 122.5 93) (width 0.6) (layer F.Cu) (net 19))
 (segment (start 122.500001 87.500001) (end 122.5 90.65) (width 0.6) (layer F.Cu) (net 19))
 (segment (start 122 87) (end 122.500001 87.500001) (width 0.6) (layer F.Cu) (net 19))
 (segment (start 122 87) (end 122 85) (width 3) (layer F.Cu) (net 19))
 (segment (start 130.5 93) (end 130.5 90.368) (width 0.6) (layer F.Cu) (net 2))
 (segment (start 130.5 90.368) (end 129.794 89.662) (width 0.6) (layer F.Cu) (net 2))
 (segment (start 129.794 89.662) (end 127.508 89.662) (width 0.6) (layer F.Cu) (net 2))
 (segment (start 125.5 87.654) (end 125.5 85.598) (width 0.6) (layer F.Cu) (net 2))
 (segment (start 127.508 89.662) (end 125.5 87.654) (width 0.6) (layer F.Cu) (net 2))
 (segment (start 125.5 85.598) (end 125.5 81.5) (width 0.6) (layer F.Cu) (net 2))
 (segment (start 127.55 81.5) (end 130.475 81.5) (width 0.6) (layer F.Cu) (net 25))
 (segment (start 123.961 118.119) (end 125.966 118.11) (width 0.6) (layer F.Cu) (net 5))
 (segment (start 122.5 116.658) (end 123.961 118.119) (width 0.6) (layer F.Cu) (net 5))
 (segment (start 122.5 109) (end 122.5 116.658) (width 0.6) (layer F.Cu) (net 5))
 (segment (start 124.5 111.35) (end 124.5 109) (width 0.6) (layer F.Cu) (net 4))
 (segment (start 125.275 114.5) (end 124.5 113.725) (width 0.6) (layer F.Cu) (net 4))
 (segment (start 124.5 113.725) (end 124.5 111.35) (width 0.6) (layer F.Cu) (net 4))
 (segment (start 125.95 114.5) (end 125.275 114.5) (width 0.6) (layer F.Cu) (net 4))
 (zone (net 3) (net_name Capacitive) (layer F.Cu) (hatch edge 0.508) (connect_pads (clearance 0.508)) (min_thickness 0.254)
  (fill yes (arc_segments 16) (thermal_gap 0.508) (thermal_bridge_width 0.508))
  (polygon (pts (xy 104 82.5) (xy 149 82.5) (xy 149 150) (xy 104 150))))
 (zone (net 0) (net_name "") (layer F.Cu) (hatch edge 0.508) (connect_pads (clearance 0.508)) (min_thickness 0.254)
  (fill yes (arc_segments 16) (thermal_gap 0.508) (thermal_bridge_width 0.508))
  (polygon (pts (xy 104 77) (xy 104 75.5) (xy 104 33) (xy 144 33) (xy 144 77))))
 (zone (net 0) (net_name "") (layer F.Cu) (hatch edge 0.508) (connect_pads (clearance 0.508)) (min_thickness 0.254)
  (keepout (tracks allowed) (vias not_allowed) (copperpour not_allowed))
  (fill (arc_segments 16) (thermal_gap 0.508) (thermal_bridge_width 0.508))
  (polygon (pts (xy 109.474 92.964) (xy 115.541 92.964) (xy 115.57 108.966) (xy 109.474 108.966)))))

